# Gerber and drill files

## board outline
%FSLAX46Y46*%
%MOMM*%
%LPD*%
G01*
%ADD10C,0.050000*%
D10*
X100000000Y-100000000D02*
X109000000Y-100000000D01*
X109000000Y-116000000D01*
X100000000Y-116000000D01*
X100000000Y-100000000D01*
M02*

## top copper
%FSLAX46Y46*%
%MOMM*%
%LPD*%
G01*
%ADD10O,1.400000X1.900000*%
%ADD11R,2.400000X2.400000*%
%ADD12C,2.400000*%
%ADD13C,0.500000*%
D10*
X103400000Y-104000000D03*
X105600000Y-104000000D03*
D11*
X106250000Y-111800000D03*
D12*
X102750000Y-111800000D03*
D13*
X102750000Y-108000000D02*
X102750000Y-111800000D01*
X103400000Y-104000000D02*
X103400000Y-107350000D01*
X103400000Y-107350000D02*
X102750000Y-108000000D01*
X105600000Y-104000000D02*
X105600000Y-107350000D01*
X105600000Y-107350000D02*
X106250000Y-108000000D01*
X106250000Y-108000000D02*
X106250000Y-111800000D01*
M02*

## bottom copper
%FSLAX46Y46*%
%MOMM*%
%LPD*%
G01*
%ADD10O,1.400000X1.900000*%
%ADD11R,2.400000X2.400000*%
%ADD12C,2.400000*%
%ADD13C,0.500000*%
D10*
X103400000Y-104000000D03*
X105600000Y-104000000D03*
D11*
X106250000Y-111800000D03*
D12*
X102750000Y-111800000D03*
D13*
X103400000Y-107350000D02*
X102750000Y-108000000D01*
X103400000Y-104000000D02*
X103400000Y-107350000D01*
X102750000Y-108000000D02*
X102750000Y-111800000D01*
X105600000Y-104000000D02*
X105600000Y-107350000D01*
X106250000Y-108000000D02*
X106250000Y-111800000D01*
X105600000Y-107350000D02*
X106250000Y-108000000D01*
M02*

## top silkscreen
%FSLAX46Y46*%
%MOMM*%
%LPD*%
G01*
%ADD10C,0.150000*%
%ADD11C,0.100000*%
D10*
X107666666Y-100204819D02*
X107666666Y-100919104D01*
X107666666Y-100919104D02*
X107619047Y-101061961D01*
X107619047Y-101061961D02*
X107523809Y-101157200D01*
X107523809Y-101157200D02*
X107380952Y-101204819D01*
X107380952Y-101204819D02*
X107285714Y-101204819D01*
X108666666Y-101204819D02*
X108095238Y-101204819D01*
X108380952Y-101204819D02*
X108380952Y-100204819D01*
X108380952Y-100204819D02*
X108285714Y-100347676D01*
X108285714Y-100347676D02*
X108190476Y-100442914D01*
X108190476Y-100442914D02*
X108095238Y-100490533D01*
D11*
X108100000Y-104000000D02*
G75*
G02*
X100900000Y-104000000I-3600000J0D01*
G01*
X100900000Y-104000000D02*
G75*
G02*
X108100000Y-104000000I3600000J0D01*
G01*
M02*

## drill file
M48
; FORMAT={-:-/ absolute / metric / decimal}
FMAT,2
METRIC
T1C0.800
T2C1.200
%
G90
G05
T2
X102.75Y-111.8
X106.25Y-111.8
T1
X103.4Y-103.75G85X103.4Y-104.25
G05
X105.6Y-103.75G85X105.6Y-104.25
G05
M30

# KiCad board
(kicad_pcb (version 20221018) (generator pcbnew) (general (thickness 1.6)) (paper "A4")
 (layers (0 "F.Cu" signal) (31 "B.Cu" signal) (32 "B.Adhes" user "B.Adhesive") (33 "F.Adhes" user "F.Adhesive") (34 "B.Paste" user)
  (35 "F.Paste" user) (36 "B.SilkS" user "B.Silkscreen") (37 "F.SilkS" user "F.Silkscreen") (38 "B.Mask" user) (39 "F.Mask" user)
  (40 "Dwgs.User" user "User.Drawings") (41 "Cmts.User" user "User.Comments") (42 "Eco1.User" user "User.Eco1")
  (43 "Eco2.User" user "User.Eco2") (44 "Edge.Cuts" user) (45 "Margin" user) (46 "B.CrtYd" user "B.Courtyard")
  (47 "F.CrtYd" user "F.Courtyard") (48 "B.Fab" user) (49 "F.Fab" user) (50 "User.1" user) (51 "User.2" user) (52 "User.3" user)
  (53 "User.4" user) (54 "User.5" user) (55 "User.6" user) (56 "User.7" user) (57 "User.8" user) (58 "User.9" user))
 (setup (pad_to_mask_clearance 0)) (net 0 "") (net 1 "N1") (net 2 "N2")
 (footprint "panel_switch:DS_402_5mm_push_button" (layer "F.Cu") (at 104.5 104)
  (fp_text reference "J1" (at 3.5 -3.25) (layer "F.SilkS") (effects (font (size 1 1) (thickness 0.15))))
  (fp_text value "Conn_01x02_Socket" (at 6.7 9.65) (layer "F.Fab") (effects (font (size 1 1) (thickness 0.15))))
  (fp_circle (center 0 0) (end 3.6 0) (stroke (width 0.1) (type default)) (fill none) (layer "F.SilkS"))
  (pad "1" thru_hole oval (at -1.1 0) (size 1.4 1.9) (drill oval 0.8 1.3) (layers "*.Cu" "*.Mask") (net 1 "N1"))
  (pad "2" thru_hole oval (at 1.1 0) (size 1.4 1.9) (drill oval 0.8 1.3) (layers "*.Cu" "*.Mask") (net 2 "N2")))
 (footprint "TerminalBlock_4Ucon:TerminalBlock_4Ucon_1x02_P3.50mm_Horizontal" (layer "B.Cu") (at 106.25 111.8 180)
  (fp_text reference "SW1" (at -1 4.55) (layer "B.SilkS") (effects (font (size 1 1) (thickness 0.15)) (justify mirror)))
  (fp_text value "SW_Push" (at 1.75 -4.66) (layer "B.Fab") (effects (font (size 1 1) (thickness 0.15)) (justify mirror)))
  (pad "1" thru_hole rect (at 0 0 180) (size 2.4 2.4) (drill 1.2) (layers "*.Cu" "*.Mask") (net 2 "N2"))
  (pad "2" thru_hole circle (at 3.5 0 180) (size 2.4 2.4) (drill 1.2) (layers "*.Cu" "*.Mask") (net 1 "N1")))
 (gr_rect (start 100 100) (end 109 116) (stroke (width 0.05) (type default)) (fill none) (layer "Edge.Cuts"))
 (segment (start 102.75 108) (end 102.75 111.8) (width 0.5) (layer "F.Cu") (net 1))
 (segment (start 103.4 104) (end 103.4 107.35) (width 0.5) (layer "F.Cu") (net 1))
 (segment (start 103.4 107.35) (end 102.75 108) (width 0.5) (layer "F.Cu") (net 1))
 (segment (start 103.4 107.35) (end 102.75 108) (width 0.5) (layer "B.Cu") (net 1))
 (segment (start 103.4 104) (end 103.4 107.35) (width 0.5) (layer "B.Cu") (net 1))
 (segment (start 102.75 108) (end 102.75 111.8) (width 0.5) (layer "B.Cu") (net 1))
 (segment (start 105.6 104) (end 105.6 107.35) (width 0.5) (layer "F.Cu") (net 2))
 (segment (start 105.6 107.35) (end 106.25 108) (width 0.5) (layer "F.Cu") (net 2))
 (segment (start 106.25 108) (end 106.25 111.8) (width 0.5) (layer "F.Cu") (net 2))
 (segment (start 105.6 104) (end 105.6 107.35) (width 0.5) (layer "B.Cu") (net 2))
 (segment (start 106.25 108) (end 106.25 111.8) (width 0.5) (layer "B.Cu") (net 2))
 (segment (start 105.6 107.35) (end 106.25 108) (width 0.5) (layer "B.Cu") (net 2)))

